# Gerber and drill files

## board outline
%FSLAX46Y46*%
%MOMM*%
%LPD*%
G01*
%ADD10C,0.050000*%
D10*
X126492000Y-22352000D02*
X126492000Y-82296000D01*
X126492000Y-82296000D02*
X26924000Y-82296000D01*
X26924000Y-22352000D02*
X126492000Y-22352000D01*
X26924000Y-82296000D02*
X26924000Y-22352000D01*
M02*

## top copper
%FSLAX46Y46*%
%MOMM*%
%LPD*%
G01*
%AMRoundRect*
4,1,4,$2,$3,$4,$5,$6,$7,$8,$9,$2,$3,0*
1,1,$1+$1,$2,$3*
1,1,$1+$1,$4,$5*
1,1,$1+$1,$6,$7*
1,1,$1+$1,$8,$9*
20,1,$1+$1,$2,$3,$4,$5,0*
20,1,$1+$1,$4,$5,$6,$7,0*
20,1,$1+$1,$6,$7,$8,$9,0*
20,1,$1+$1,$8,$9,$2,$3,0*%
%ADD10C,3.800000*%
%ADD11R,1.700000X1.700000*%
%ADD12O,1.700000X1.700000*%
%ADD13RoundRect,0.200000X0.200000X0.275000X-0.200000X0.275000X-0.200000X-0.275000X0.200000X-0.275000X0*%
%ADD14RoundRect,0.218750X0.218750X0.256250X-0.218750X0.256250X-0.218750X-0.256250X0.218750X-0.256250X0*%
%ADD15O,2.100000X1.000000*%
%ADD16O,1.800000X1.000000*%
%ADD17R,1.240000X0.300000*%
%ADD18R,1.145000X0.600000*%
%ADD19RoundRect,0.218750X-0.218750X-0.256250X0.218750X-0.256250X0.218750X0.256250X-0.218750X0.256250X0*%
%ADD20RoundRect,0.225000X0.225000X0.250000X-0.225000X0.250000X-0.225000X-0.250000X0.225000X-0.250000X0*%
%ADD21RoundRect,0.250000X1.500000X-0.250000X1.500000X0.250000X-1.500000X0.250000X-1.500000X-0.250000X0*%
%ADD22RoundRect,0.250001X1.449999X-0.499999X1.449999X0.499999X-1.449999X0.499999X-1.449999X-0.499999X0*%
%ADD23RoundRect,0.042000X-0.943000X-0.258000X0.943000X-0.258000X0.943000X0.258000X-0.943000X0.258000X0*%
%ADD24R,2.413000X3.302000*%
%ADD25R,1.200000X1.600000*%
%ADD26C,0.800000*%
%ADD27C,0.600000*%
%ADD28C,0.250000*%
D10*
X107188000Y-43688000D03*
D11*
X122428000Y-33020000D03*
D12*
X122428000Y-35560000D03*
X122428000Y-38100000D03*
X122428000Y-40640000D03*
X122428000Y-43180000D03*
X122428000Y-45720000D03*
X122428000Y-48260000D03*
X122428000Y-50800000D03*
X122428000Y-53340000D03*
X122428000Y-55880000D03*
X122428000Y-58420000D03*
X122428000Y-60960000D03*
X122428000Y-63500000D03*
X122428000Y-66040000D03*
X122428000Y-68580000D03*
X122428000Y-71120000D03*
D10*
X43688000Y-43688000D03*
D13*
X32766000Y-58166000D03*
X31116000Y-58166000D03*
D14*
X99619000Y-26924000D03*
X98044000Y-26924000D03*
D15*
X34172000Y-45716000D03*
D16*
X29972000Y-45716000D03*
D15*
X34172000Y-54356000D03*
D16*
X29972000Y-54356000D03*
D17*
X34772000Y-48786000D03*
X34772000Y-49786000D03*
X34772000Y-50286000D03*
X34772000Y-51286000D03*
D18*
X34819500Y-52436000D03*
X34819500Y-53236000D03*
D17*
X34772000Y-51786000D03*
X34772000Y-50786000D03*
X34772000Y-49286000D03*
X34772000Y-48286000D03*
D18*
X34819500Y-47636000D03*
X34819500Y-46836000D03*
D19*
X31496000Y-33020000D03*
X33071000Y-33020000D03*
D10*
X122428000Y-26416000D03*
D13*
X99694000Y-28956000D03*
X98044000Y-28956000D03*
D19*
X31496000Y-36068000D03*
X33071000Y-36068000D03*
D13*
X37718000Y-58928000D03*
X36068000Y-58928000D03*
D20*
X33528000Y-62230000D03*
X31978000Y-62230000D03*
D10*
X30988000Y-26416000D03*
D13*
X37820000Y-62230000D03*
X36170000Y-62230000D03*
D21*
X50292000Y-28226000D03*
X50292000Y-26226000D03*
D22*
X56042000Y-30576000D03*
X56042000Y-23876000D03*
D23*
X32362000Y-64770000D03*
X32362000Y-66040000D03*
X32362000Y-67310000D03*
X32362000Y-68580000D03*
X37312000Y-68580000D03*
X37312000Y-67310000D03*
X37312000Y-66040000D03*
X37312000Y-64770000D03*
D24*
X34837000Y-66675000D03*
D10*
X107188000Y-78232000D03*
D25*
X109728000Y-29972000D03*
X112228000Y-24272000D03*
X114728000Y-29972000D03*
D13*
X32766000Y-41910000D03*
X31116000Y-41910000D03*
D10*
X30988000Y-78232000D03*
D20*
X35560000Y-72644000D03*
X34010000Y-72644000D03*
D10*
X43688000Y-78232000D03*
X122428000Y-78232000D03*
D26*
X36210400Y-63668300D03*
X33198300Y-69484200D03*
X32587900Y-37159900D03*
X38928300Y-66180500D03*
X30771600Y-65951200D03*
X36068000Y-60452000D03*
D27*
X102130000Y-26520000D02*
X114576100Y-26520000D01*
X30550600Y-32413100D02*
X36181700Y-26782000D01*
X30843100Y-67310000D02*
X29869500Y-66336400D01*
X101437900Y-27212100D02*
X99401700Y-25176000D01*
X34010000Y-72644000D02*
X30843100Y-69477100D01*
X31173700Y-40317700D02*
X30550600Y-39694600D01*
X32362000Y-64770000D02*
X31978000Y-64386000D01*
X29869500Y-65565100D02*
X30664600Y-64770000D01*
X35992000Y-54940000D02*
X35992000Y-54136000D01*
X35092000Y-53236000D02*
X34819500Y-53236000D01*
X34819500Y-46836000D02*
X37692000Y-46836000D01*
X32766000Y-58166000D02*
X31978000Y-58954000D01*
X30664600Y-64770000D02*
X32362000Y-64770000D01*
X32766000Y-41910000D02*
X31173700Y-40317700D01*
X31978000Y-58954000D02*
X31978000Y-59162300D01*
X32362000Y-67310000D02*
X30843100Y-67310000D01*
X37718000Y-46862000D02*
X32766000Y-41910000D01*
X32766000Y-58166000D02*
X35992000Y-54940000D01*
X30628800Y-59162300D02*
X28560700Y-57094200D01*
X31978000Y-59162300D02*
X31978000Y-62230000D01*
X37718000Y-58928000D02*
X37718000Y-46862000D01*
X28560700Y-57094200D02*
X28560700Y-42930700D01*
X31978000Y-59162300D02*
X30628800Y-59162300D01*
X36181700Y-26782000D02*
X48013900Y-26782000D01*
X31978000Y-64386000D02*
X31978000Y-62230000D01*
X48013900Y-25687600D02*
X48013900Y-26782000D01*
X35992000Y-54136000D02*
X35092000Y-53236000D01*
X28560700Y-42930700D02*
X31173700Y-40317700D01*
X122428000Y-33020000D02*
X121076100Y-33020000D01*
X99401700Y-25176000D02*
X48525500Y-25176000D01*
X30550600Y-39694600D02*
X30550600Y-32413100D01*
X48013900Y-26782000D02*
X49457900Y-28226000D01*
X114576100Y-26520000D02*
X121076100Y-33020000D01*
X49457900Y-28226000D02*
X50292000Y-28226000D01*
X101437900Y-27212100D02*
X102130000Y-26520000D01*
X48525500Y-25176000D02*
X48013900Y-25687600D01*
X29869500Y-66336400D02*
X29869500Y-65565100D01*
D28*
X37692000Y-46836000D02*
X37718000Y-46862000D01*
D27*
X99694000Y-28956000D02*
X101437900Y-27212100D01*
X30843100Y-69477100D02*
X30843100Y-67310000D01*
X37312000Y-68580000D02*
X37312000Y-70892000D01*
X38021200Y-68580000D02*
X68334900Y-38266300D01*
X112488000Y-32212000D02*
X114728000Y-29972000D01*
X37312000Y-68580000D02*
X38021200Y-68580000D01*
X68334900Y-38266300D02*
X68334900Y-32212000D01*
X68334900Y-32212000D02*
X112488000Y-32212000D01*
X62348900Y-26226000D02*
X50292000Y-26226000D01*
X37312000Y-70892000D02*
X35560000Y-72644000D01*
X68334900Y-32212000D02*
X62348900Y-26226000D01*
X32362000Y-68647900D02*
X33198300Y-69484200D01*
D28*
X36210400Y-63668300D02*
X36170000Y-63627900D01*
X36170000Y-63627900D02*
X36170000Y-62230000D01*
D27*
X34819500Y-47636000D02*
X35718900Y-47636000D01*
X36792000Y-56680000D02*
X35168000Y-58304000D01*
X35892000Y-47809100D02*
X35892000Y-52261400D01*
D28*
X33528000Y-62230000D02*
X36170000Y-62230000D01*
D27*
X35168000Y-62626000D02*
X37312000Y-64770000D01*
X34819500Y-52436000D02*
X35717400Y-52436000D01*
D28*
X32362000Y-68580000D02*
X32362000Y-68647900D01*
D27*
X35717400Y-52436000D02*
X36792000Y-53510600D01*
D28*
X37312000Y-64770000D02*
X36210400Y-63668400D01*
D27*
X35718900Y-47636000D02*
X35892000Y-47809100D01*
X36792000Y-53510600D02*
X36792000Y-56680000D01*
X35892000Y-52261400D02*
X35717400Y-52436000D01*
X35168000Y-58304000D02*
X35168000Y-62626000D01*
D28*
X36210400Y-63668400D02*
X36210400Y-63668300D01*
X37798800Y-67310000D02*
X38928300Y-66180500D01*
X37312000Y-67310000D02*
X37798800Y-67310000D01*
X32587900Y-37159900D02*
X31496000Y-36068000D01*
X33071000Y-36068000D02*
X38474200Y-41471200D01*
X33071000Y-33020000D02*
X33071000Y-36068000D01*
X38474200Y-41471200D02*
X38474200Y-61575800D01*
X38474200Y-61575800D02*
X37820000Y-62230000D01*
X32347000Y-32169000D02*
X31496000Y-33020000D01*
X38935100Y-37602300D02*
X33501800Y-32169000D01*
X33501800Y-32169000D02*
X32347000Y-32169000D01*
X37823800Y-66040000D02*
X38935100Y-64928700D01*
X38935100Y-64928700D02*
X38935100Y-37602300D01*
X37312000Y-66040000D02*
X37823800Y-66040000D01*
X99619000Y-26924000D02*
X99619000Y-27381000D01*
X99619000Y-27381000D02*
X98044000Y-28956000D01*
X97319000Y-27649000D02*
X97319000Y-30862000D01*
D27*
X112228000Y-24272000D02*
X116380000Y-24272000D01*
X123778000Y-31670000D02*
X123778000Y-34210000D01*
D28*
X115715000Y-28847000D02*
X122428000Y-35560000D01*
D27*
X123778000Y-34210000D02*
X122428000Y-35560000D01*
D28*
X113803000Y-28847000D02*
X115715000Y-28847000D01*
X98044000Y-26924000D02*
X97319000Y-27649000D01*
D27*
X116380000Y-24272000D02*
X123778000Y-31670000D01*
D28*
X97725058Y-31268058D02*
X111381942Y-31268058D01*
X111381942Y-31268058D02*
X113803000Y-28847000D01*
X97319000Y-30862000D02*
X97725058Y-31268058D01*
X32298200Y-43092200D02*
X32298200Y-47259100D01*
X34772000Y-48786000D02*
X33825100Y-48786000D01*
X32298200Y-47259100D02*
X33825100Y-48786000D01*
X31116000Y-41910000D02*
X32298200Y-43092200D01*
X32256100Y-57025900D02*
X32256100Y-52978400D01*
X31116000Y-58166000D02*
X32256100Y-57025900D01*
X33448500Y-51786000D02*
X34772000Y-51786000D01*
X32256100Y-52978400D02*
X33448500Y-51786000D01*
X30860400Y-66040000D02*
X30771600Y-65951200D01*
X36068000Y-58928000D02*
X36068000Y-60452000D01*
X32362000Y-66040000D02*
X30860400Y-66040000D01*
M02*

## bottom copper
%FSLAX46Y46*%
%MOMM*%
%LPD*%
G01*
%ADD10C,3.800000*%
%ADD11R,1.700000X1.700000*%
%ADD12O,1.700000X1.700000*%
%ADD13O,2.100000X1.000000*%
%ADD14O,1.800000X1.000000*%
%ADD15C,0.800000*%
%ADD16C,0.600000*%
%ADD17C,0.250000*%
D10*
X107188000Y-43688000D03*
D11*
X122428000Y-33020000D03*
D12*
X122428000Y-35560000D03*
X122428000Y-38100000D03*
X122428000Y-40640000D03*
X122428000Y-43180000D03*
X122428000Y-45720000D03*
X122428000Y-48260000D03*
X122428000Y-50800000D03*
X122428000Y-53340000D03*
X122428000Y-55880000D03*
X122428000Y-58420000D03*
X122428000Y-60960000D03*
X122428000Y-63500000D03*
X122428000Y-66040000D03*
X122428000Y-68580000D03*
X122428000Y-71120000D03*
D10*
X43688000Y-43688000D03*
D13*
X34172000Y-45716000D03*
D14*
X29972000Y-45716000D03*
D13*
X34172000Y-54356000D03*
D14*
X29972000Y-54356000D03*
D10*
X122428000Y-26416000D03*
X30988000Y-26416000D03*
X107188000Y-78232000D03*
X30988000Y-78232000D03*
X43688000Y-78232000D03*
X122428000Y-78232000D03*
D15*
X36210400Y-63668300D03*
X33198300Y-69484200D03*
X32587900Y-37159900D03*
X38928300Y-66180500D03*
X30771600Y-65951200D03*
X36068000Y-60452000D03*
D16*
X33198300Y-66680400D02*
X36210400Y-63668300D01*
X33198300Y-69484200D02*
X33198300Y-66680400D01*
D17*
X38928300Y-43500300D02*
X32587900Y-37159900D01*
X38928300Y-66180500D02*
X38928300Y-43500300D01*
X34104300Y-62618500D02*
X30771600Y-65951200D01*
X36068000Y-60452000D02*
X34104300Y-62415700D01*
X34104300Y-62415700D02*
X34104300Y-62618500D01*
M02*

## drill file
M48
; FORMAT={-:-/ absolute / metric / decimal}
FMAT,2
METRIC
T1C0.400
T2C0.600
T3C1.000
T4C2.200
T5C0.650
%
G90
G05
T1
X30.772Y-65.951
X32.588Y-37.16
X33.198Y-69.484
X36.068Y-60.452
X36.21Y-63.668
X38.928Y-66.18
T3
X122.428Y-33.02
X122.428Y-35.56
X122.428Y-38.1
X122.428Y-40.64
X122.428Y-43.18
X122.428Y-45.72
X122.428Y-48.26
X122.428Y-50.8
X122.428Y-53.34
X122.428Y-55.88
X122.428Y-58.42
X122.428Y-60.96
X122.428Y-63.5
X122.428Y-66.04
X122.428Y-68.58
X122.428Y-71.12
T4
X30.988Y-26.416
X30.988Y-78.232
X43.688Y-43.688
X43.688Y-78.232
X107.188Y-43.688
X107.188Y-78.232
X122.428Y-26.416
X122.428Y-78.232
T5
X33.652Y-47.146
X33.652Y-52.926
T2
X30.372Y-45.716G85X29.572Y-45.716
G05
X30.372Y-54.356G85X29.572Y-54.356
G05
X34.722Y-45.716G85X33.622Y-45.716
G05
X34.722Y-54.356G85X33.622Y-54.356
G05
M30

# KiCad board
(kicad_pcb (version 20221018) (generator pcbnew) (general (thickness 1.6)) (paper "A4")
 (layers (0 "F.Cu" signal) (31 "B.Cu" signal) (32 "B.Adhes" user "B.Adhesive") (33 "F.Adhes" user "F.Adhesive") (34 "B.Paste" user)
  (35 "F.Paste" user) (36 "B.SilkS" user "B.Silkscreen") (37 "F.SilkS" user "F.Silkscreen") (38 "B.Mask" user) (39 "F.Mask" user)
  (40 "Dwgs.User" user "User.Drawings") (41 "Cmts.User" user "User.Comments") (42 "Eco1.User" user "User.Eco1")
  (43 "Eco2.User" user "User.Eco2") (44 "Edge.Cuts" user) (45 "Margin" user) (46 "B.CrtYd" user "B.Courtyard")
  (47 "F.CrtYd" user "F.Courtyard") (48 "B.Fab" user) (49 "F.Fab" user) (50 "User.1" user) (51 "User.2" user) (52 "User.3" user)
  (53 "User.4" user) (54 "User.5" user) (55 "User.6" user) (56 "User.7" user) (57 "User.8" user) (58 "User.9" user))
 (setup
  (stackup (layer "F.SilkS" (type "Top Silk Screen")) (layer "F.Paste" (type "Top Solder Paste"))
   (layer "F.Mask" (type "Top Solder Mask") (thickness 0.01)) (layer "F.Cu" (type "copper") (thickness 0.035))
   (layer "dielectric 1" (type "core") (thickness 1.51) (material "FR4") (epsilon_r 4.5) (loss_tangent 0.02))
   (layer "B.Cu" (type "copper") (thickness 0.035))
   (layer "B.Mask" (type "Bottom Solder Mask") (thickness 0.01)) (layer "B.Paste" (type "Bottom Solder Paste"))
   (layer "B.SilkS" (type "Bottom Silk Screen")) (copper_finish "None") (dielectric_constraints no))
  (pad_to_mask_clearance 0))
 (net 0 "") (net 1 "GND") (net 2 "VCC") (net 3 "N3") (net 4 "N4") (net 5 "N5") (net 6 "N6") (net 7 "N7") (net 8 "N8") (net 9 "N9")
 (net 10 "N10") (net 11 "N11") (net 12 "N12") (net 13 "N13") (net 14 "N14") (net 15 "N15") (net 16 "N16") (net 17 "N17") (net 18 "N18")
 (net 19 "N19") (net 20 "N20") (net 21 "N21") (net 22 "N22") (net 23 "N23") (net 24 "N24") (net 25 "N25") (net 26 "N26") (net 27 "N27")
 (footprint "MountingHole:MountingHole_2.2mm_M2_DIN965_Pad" (layer "F.Cu") (at 107.188 43.688)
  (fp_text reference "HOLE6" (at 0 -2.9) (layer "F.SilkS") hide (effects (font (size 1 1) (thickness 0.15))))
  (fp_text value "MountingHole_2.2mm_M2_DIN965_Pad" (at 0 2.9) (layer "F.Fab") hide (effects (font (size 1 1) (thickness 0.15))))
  (pad "1" thru_hole circle (at 0 0) (size 3.8 3.8) (drill 2.2) (layers "*.Cu" "*.Mask")))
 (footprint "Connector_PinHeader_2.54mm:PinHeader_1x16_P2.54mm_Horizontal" (layer "F.Cu") (at 122.428 33.02)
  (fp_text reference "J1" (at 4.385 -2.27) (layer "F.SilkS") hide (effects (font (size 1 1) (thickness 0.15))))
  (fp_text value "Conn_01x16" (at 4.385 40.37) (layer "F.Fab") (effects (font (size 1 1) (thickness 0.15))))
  (pad "1" thru_hole rect (at 0 0) (size 1.7 1.7) (drill 1) (layers "*.Cu" "*.Mask") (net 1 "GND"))
  (pad "2" thru_hole oval (at 0 2.54) (size 1.7 1.7) (drill 1) (layers "*.Cu" "*.Mask") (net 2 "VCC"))
  (pad "3" thru_hole oval (at 0 5.08) (size 1.7 1.7) (drill 1) (layers "*.Cu" "*.Mask") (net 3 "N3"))
  (pad "4" thru_hole oval (at 0 7.62) (size 1.7 1.7) (drill 1) (layers "*.Cu" "*.Mask") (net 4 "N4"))
  (pad "5" thru_hole oval (at 0 10.16) (size 1.7 1.7) (drill 1) (layers "*.Cu" "*.Mask") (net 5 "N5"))
  (pad "6" thru_hole oval (at 0 12.7) (size 1.7 1.7) (drill 1) (layers "*.Cu" "*.Mask") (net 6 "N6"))
  (pad "7" thru_hole oval (at 0 15.24) (size 1.7 1.7) (drill 1) (layers "*.Cu" "*.Mask") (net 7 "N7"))
  (pad "8" thru_hole oval (at 0 17.78) (size 1.7 1.7) (drill 1) (layers "*.Cu" "*.Mask") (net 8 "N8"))
  (pad "9" thru_hole oval (at 0 20.32) (size 1.7 1.7) (drill 1) (layers "*.Cu" "*.Mask") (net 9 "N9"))
  (pad "10" thru_hole oval (at 0 22.86) (size 1.7 1.7) (drill 1) (layers "*.Cu" "*.Mask") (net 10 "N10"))
  (pad "11" thru_hole oval (at 0 25.4) (size 1.7 1.7) (drill 1) (layers "*.Cu" "*.Mask") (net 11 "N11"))
  (pad "12" thru_hole oval (at 0 27.94) (size 1.7 1.7) (drill 1) (layers "*.Cu" "*.Mask") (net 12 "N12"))
  (pad "13" thru_hole oval (at 0 30.48) (size 1.7 1.7) (drill 1) (layers "*.Cu" "*.Mask") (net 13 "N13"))
  (pad "14" thru_hole oval (at 0 33.02) (size 1.7 1.7) (drill 1) (layers "*.Cu" "*.Mask") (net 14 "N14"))
  (pad "15" thru_hole oval (at 0 35.56) (size 1.7 1.7) (drill 1) (layers "*.Cu" "*.Mask") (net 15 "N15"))
  (pad "16" thru_hole oval (at 0 38.1) (size 1.7 1.7) (drill 1) (layers "*.Cu" "*.Mask") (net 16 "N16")))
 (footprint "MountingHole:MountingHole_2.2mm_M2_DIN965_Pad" (layer "F.Cu") (at 43.688 43.688)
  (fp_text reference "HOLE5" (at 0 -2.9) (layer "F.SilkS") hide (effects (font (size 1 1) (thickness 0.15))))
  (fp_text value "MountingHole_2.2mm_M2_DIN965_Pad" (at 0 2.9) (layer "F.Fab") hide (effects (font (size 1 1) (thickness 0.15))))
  (pad "1" thru_hole circle (at 0 0) (size 3.8 3.8) (drill 2.2) (layers "*.Cu" "*.Mask")))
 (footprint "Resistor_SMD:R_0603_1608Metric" (layer "F.Cu") (at 31.941 58.166 180)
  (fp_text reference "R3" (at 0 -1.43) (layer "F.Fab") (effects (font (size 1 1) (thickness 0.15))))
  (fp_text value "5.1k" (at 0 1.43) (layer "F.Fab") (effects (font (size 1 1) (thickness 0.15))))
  (pad "1" smd roundrect (at -0.825 0 180) (size 0.8 0.95) (layers "F.Cu" "F.Paste" "F.Mask") (roundrect_rratio 0.25) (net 1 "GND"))
  (pad "2" smd roundrect (at 0.825 0 180) (size 0.8 0.95) (layers "F.Cu" "F.Paste" "F.Mask") (roundrect_rratio 0.25) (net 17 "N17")))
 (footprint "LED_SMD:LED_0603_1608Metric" (layer "F.Cu") (at 98.8315 26.924 180)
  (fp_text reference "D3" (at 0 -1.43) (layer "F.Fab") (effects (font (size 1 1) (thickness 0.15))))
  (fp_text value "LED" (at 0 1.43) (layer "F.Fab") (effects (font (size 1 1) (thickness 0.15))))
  (pad "1" smd roundrect (at -0.7875 0 180) (size 0.875 0.95) (layers "F.Cu" "F.Paste" "F.Mask") (roundrect_rratio 0.25) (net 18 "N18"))
  (pad "2" smd roundrect (at 0.7875 0 180) (size 0.875 0.95) (layers "F.Cu" "F.Paste" "F.Mask") (roundrect_rratio 0.25) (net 2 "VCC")))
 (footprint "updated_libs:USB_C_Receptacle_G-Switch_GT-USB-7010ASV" (layer "F.Cu") (at 31.047 50.036 -90)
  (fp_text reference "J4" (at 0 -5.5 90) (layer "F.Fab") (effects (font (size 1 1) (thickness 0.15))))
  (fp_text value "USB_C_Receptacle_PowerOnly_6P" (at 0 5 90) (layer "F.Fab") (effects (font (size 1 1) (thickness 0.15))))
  (pad "" thru_hole oval (at -4.32 -3.125 270) (size 1 2.1) (drill oval 0.6 1.7) (layers "*.Cu" "*.Mask"))
  (pad "" thru_hole oval (at -4.32 1.075 270) (size 1 1.8) (drill oval 0.6 1.4) (layers "*.Cu" "*.Mask"))
  (pad "" np_thru_hole circle (at -2.89 -2.605 270) (size 0.65 0.65) (drill 0.65) (layers "*.Cu" "*.Mask"))
  (pad "" np_thru_hole circle (at 2.89 -2.605 270) (size 0.65 0.65) (drill 0.65) (layers "*.Cu" "*.Mask"))
  (pad "" thru_hole oval (at 4.32 -3.125 270) (size 1 2.1) (drill oval 0.6 1.7) (layers "*.Cu" "*.Mask"))
  (pad "" thru_hole oval (at 4.32 1.075 270) (size 1 1.8) (drill oval 0.6 1.4) (layers "*.Cu" "*.Mask"))
  (pad "A5" smd rect (at -1.25 -3.725 270) (size 0.3 1.24) (layers "F.Cu" "F.Paste" "F.Mask") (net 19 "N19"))
  (pad "A6" smd rect (at -0.25 -3.725 270) (size 0.3 1.24) (layers "F.Cu" "F.Paste" "F.Mask"))
  (pad "A7" smd rect (at 0.25 -3.725 270) (size 0.3 1.24) (layers "F.Cu" "F.Paste" "F.Mask"))
  (pad "A8" smd rect (at 1.25 -3.725 270) (size 0.3 1.24) (layers "F.Cu" "F.Paste" "F.Mask"))
  (pad "A9" smd rect (at 2.4 -3.7725 270) (size 0.6 1.145) (layers "F.Cu" "F.Paste" "F.Mask") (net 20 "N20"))
  (pad "A12" smd rect (at 3.2 -3.7725 270) (size 0.6 1.145) (layers "F.Cu" "F.Paste" "F.Mask") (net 1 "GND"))
  (pad "B5" smd rect (at 1.75 -3.725 270) (size 0.3 1.24) (layers "F.Cu" "F.Paste" "F.Mask") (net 17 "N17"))
  (pad "B6" smd rect (at 0.75 -3.725 270) (size 0.3 1.24) (layers "F.Cu" "F.Paste" "F.Mask"))
  (pad "B7" smd rect (at -0.75 -3.725 270) (size 0.3 1.24) (layers "F.Cu" "F.Paste" "F.Mask"))
  (pad "B8" smd rect (at -1.75 -3.725 270) (size 0.3 1.24) (layers "F.Cu" "F.Paste" "F.Mask"))
  (pad "B9" smd rect (at -2.4 -3.7725 270) (size 0.6 1.145) (layers "F.Cu" "F.Paste" "F.Mask") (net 20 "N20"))
  (pad "B12" smd rect (at -3.2 -3.7725 270) (size 0.6 1.145) (layers "F.Cu" "F.Paste" "F.Mask") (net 1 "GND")))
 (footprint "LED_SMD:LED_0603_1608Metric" (layer "F.Cu") (at 32.2835 33.02)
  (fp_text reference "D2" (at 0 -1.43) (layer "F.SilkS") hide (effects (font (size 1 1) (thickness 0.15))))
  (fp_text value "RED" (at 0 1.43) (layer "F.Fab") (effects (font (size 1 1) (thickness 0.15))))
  (pad "1" smd roundrect (at -0.7875 0) (size 0.875 0.95) (layers "F.Cu" "F.Paste" "F.Mask") (roundrect_rratio 0.25) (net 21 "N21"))
  (pad "2" smd roundrect (at 0.7875 0) (size 0.875 0.95) (layers "F.Cu" "F.Paste" "F.Mask") (roundrect_rratio 0.25) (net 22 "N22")))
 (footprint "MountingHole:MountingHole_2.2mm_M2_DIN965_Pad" (layer "F.Cu") (at 122.428 26.416)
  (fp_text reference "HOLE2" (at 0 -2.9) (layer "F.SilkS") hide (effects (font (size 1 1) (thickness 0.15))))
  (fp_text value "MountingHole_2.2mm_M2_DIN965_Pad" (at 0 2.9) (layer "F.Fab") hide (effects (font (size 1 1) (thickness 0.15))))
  (pad "1" thru_hole circle (at 0 0) (size 3.8 3.8) (drill 2.2) (layers "*.Cu" "*.Mask")))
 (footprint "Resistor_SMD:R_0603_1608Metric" (layer "F.Cu") (at 98.869 28.956 180)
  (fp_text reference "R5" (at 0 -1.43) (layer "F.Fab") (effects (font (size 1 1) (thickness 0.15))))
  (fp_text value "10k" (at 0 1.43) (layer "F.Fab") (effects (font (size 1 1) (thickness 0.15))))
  (pad "1" smd roundrect (at -0.825 0 180) (size 0.8 0.95) (layers "F.Cu" "F.Paste" "F.Mask") (roundrect_rratio 0.25) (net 1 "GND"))
  (pad "2" smd roundrect (at 0.825 0 180) (size 0.8 0.95) (layers "F.Cu" "F.Paste" "F.Mask") (roundrect_rratio 0.25) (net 18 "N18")))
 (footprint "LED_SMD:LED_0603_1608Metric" (layer "F.Cu") (at 32.2835 36.068)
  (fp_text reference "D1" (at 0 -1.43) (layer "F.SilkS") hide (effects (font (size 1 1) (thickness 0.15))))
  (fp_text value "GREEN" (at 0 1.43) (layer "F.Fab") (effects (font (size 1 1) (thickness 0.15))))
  (pad "1" smd roundrect (at -0.7875 0) (size 0.875 0.95) (layers "F.Cu" "F.Paste" "F.Mask") (roundrect_rratio 0.25) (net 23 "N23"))
  (pad "2" smd roundrect (at 0.7875 0) (size 0.875 0.95) (layers "F.Cu" "F.Paste" "F.Mask") (roundrect_rratio 0.25) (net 22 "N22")))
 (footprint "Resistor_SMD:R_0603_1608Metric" (layer "F.Cu") (at 36.893 58.928 180)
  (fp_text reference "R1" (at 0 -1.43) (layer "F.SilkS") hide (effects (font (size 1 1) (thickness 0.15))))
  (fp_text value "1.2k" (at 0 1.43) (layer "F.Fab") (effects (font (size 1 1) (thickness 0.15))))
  (pad "1" smd roundrect (at -0.825 0 180) (size 0.8 0.95) (layers "F.Cu" "F.Paste" "F.Mask") (roundrect_rratio 0.25) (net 1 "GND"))
  (pad "2" smd roundrect (at 0.825 0 180) (size 0.8 0.95) (layers "F.Cu" "F.Paste" "F.Mask") (roundrect_rratio 0.25) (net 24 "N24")))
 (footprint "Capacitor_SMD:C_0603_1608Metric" (layer "F.Cu") (at 32.753 62.23 180)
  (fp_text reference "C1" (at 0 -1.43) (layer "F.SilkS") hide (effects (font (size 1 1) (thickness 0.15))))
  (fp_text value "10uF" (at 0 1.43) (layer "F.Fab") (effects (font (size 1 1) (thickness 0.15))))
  (pad "1" smd roundrect (at -0.775 0 180) (size 0.9 0.95) (layers "F.Cu" "F.Paste" "F.Mask") (roundrect_rratio 0.25) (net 20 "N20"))
  (pad "2" smd roundrect (at 0.775 0 180) (size 0.9 0.95) (layers "F.Cu" "F.Paste" "F.Mask") (roundrect_rratio 0.25) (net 1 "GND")))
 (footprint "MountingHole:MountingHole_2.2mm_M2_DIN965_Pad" (layer "F.Cu") (at 30.988 26.416)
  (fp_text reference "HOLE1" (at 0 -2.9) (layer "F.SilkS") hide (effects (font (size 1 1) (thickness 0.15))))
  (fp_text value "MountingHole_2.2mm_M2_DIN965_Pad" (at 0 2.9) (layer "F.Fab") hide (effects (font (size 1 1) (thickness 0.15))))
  (pad "1" thru_hole circle (at 0 0) (size 3.8 3.8) (drill 2.2) (layers "*.Cu" "*.Mask")))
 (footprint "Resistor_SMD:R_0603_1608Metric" (layer "F.Cu") (at 36.995 62.23 180)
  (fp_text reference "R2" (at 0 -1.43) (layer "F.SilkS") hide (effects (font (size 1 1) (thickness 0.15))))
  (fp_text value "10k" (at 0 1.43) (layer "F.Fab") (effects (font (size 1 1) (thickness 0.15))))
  (pad "1" smd roundrect (at -0.825 0 180) (size 0.8 0.95) (layers "F.Cu" "F.Paste" "F.Mask") (roundrect_rratio 0.25) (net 22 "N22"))
  (pad "2" smd roundrect (at 0.825 0 180) (size 0.8 0.95) (layers "F.Cu" "F.Paste" "F.Mask") (roundrect_rratio 0.25) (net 20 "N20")))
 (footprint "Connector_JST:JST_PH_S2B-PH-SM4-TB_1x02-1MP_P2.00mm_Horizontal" (layer "F.Cu") (at 53.142 27.226 90)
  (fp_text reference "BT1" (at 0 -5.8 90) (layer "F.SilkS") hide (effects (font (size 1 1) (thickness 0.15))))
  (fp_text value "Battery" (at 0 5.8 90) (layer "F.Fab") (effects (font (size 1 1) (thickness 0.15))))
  (pad "1" smd roundrect (at -1 -2.85 90) (size 1 3.5) (layers "F.Cu" "F.Paste" "F.Mask") (roundrect_rratio 0.25) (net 1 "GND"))
  (pad "2" smd roundrect (at 1 -2.85 90) (size 1 3.5) (layers "F.Cu" "F.Paste" "F.Mask") (roundrect_rratio 0.25) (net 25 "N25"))
  (pad "MP" smd roundrect (at -3.35 2.9 90) (size 1.5 3.4) (layers "F.Cu" "F.Paste" "F.Mask") (roundrect_rratio 0.1666673333))
  (pad "MP" smd roundrect (at 3.35 2.9 90) (size 1.5 3.4) (layers "F.Cu" "F.Paste" "F.Mask") (roundrect_rratio 0.1666673333)))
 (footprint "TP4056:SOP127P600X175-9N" (layer "F.Cu") (at 34.837 66.675)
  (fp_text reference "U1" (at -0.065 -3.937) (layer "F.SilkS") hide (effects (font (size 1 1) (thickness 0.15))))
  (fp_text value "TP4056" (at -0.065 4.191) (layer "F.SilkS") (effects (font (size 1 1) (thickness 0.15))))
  (pad "1" smd roundrect (at -2.475 -1.905) (size 1.97 0.6) (layers "F.Cu" "F.Paste" "F.Mask") (roundrect_rratio 0.07) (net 1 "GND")
   (solder_mask_margin 0.102))
  (pad "2" smd roundrect (at -2.475 -0.635) (size 1.97 0.6) (layers "F.Cu" "F.Paste" "F.Mask") (roundrect_rratio 0.07) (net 24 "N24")
   (solder_mask_margin 0.102))
  (pad "3" smd roundrect (at -2.475 0.635) (size 1.97 0.6) (layers "F.Cu" "F.Paste" "F.Mask") (roundrect_rratio 0.07) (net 1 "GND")
   (solder_mask_margin 0.102))
  (pad "4" smd roundrect (at -2.475 1.905) (size 1.97 0.6) (layers "F.Cu" "F.Paste" "F.Mask") (roundrect_rratio 0.07) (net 20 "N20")
   (solder_mask_margin 0.102))
  (pad "5" smd roundrect (at 2.475 1.905) (size 1.97 0.6) (layers "F.Cu" "F.Paste" "F.Mask") (roundrect_rratio 0.07) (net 25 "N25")
   (solder_mask_margin 0.102))
  (pad "6" smd roundrect (at 2.475 0.635) (size 1.97 0.6) (layers "F.Cu" "F.Paste" "F.Mask") (roundrect_rratio 0.07) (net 23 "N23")
   (solder_mask_margin 0.102))
  (pad "7" smd roundrect (at 2.475 -0.635) (size 1.97 0.6) (layers "F.Cu" "F.Paste" "F.Mask") (roundrect_rratio 0.07) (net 21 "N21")
   (solder_mask_margin 0.102))
  (pad "8" smd roundrect (at 2.475 -1.905) (size 1.97 0.6) (layers "F.Cu" "F.Paste" "F.Mask") (roundrect_rratio 0.07) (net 20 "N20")
   (solder_mask_margin 0.102))
  (pad "9" smd rect (at 0 0) (size 2.413 3.302) (layers "F.Cu" "F.Mask") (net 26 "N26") (solder_mask_margin 0.102)))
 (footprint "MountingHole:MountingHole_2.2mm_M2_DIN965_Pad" (layer "F.Cu") (at 107.188 78.232)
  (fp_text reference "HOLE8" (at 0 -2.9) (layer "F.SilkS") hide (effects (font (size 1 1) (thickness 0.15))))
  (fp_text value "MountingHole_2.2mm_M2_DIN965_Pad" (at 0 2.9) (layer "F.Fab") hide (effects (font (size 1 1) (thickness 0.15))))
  (pad "1" thru_hole circle (at 0 0) (size 3.8 3.8) (drill 2.2) (layers "*.Cu" "*.Mask")))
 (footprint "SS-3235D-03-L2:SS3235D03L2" (layer "F.Cu") (at 112.228 27.122)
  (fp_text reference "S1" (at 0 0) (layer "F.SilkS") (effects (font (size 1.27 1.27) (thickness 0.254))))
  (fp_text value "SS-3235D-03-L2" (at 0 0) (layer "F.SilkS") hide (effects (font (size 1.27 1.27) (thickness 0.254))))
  (pad "1" smd rect (at -2.5 2.85) (size 1.2 1.6) (layers "F.Cu" "F.Paste" "F.Mask") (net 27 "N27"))
  (pad "2" smd rect (at 0 -2.85) (size 1.2 1.6) (layers "F.Cu" "F.Paste" "F.Mask") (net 2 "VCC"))
  (pad "3" smd rect (at 2.5 2.85) (size 1.2 1.6) (layers "F.Cu" "F.Paste" "F.Mask") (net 25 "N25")))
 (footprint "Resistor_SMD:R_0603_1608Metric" (layer "F.Cu") (at 31.941 41.91 180)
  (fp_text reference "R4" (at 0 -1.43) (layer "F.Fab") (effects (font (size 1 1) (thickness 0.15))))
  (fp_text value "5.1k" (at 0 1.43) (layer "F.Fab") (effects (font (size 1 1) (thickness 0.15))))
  (pad "1" smd roundrect (at -0.825 0 180) (size 0.8 0.95) (layers "F.Cu" "F.Paste" "F.Mask") (roundrect_rratio 0.25) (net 1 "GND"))
  (pad "2" smd roundrect (at 0.825 0 180) (size 0.8 0.95) (layers "F.Cu" "F.Paste" "F.Mask") (roundrect_rratio 0.25) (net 19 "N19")))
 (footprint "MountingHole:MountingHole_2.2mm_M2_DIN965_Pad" (layer "F.Cu") (at 30.988 78.232)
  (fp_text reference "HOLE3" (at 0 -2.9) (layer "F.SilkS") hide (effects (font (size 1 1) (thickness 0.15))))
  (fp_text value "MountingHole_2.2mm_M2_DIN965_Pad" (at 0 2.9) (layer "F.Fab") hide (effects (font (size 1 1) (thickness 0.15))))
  (pad "1" thru_hole circle (at 0 0) (size 3.8 3.8) (drill 2.2) (layers "*.Cu" "*.Mask")))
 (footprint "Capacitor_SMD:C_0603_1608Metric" (layer "F.Cu") (at 34.785 72.644 180)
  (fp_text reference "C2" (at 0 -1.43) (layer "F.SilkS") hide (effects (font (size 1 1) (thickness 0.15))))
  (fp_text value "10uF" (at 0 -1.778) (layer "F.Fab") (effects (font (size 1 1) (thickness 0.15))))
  (pad "1" smd roundrect (at -0.775 0 180) (size 0.9 0.95) (layers "F.Cu" "F.Paste" "F.Mask") (roundrect_rratio 0.25) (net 25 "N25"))
  (pad "2" smd roundrect (at 0.775 0 180) (size 0.9 0.95) (layers "F.Cu" "F.Paste" "F.Mask") (roundrect_rratio 0.25) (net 1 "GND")))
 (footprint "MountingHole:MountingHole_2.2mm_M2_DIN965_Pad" (layer "F.Cu") (at 43.688 78.232)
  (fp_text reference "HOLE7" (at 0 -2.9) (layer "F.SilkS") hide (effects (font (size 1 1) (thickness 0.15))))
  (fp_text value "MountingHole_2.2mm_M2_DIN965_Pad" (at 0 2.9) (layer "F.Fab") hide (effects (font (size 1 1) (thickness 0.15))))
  (pad "1" thru_hole circle (at 0 0) (size 3.8 3.8) (drill 2.2) (layers "*.Cu" "*.Mask")))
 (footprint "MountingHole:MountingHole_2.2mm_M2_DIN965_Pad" (layer "F.Cu") (at 122.428 78.232)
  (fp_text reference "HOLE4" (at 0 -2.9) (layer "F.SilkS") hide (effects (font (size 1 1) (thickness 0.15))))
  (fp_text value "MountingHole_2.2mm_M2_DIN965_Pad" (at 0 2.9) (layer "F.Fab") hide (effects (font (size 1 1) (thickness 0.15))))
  (pad "1" thru_hole circle (at 0 0) (size 3.8 3.8) (drill 2.2) (layers "*.Cu" "*.Mask")))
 (gr_line (start 126.492 22.352) (end 126.492 82.296) (stroke (width 0.05) (type solid)) (layer "Edge.Cuts"))
 (gr_line (start 126.492 82.296) (end 26.924 82.296) (stroke (width 0.05) (type solid)) (layer "Edge.Cuts"))
 (gr_line (start 26.924 22.352) (end 126.492 22.352) (stroke (width 0.05) (type solid)) (layer "Edge.Cuts"))
 (gr_line (start 26.924 82.296) (end 26.924 22.352) (stroke (width 0.05) (type solid)) (layer "Edge.Cuts"))
 (segment (start 102.13 26.52) (end 114.5761 26.52) (width 0.6) (layer "F.Cu") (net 1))
 (segment (start 30.5506 32.4131) (end 36.1817 26.782) (width 0.6) (layer "F.Cu") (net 1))
 (segment (start 30.8431 67.31) (end 29.8695 66.3364) (width 0.6) (layer "F.Cu") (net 1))
 (segment (start 101.4379 27.2121) (end 99.4017 25.176) (width 0.6) (layer "F.Cu") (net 1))
 (segment (start 34.01 72.644) (end 30.8431 69.4771) (width 0.6) (layer "F.Cu") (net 1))
 (segment (start 31.1737 40.3177) (end 30.5506 39.6946) (width 0.6) (layer "F.Cu") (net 1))
 (segment (start 32.362 64.77) (end 31.978 64.386) (width 0.6) (layer "F.Cu") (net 1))
 (segment (start 29.8695 65.5651) (end 30.6646 64.77) (width 0.6) (layer "F.Cu") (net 1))
 (segment (start 35.992 54.94) (end 35.992 54.136) (width 0.6) (layer "F.Cu") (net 1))
 (segment (start 35.092 53.236) (end 34.8195 53.236) (width 0.6) (layer "F.Cu") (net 1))
 (segment (start 34.8195 46.836) (end 37.692 46.836) (width 0.6) (layer "F.Cu") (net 1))
 (segment (start 32.766 58.166) (end 31.978 58.954) (width 0.6) (layer "F.Cu") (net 1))
 (segment (start 30.6646 64.77) (end 32.362 64.77) (width 0.6) (layer "F.Cu") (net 1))
 (segment (start 32.766 41.91) (end 31.1737 40.3177) (width 0.6) (layer "F.Cu") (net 1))
 (segment (start 31.978 58.954) (end 31.978 59.1623) (width 0.6) (layer "F.Cu") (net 1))
 (segment (start 32.362 67.31) (end 30.8431 67.31) (width 0.6) (layer "F.Cu") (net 1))
 (segment (start 37.718 46.862) (end 32.766 41.91) (width 0.6) (layer "F.Cu") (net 1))
 (segment (start 32.766 58.166) (end 35.992 54.94) (width 0.6) (layer "F.Cu") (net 1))
 (segment (start 30.6288 59.1623) (end 28.5607 57.0942) (width 0.6) (layer "F.Cu") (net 1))
 (segment (start 31.978 59.1623) (end 31.978 62.23) (width 0.6) (layer "F.Cu") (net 1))
 (segment (start 37.718 58.928) (end 37.718 46.862) (width 0.6) (layer "F.Cu") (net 1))
 (segment (start 28.5607 57.0942) (end 28.5607 42.9307) (width 0.6) (layer "F.Cu") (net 1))
 (segment (start 31.978 59.1623) (end 30.6288 59.1623) (width 0.6) (layer "F.Cu") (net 1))
 (segment (start 36.1817 26.782) (end 48.0139 26.782) (width 0.6) (layer "F.Cu") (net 1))
 (segment (start 31.978 64.386) (end 31.978 62.23) (width 0.6) (layer "F.Cu") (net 1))
 (segment (start 48.0139 25.6876) (end 48.0139 26.782) (width 0.6) (layer "F.Cu") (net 1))
 (segment (start 35.992 54.136) (end 35.092 53.236) (width 0.6) (layer "F.Cu") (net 1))
 (segment (start 28.5607 42.9307) (end 31.1737 40.3177) (width 0.6) (layer "F.Cu") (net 1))
 (segment (start 122.428 33.02) (end 121.0761 33.02) (width 0.6) (layer "F.Cu") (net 1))
 (segment (start 99.4017 25.176) (end 48.5255 25.176) (width 0.6) (layer "F.Cu") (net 1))
 (segment (start 30.5506 39.6946) (end 30.5506 32.4131) (width 0.6) (layer "F.Cu") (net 1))
 (segment (start 48.0139 26.782) (end 49.4579 28.226) (width 0.6) (layer "F.Cu") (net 1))
 (segment (start 114.5761 26.52) (end 121.0761 33.02) (width 0.6) (layer "F.Cu") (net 1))
 (segment (start 49.4579 28.226) (end 50.292 28.226) (width 0.6) (layer "F.Cu") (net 1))
 (segment (start 101.4379 27.2121) (end 102.13 26.52) (width 0.6) (layer "F.Cu") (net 1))
 (segment (start 48.5255 25.176) (end 48.0139 25.6876) (width 0.6) (layer "F.Cu") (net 1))
 (segment (start 29.8695 66.3364) (end 29.8695 65.5651) (width 0.6) (layer "F.Cu") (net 1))
 (segment (start 37.692 46.836) (end 37.718 46.862) (width 0.25) (layer "F.Cu") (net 1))
 (segment (start 99.694 28.956) (end 101.4379 27.2121) (width 0.6) (layer "F.Cu") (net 1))
 (segment (start 30.8431 69.4771) (end 30.8431 67.31) (width 0.6) (layer "F.Cu") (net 1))
 (segment (start 37.312 68.58) (end 37.312 70.892) (width 0.6) (layer "F.Cu") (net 25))
 (segment (start 38.0212 68.58) (end 68.3349 38.2663) (width 0.6) (layer "F.Cu") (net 25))
 (segment (start 112.488 32.212) (end 114.728 29.972) (width 0.6) (layer "F.Cu") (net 25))
 (segment (start 37.312 68.58) (end 38.0212 68.58) (width 0.6) (layer "F.Cu") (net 25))
 (segment (start 68.3349 38.2663) (end 68.3349 32.212) (width 0.6) (layer "F.Cu") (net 25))
 (segment (start 68.3349 32.212) (end 112.488 32.212) (width 0.6) (layer "F.Cu") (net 25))
 (segment (start 62.3489 26.226) (end 50.292 26.226) (width 0.6) (layer "F.Cu") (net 25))
 (segment (start 37.312 70.892) (end 35.56 72.644) (width 0.6) (layer "F.Cu") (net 25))
 (segment (start 68.3349 32.212) (end 62.3489 26.226) (width 0.6) (layer "F.Cu") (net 25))
 (segment (start 32.362 68.6479) (end 33.1983 69.4842) (width 0.6) (layer "F.Cu") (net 20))
 (segment (start 36.2104 63.6683) (end 36.17 63.6279) (width 0.25) (layer "F.Cu") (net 20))
 (segment (start 36.17 63.6279) (end 36.17 62.23) (width 0.25) (layer "F.Cu") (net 20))
 (segment (start 34.8195 47.636) (end 35.7189 47.636) (width 0.6) (layer "F.Cu") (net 20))
 (segment (start 36.792 56.68) (end 35.168 58.304) (width 0.6) (layer "F.Cu") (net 20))
 (segment (start 35.892 47.8091) (end 35.892 52.2614) (width 0.6) (layer "F.Cu") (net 20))
 (segment (start 33.528 62.23) (end 36.17 62.23) (width 0.25) (layer "F.Cu") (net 20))
 (segment (start 35.168 62.626) (end 37.312 64.77) (width 0.6) (layer "F.Cu") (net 20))
 (segment (start 34.8195 52.436) (end 35.7174 52.436) (width 0.6) (layer "F.Cu") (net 20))
 (segment (start 32.362 68.58) (end 32.362 68.6479) (width 0.25) (layer "F.Cu") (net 20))
 (segment (start 35.7174 52.436) (end 36.792 53.5106) (width 0.6) (layer "F.Cu") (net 20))
 (segment (start 37.312 64.77) (end 36.2104 63.6684) (width 0.25) (layer "F.Cu") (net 20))
 (segment (start 35.7189 47.636) (end 35.892 47.8091) (width 0.6) (layer "F.Cu") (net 20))
 (segment (start 36.792 53.5106) (end 36.792 56.68) (width 0.6) (layer "F.Cu") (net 20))
 (segment (start 35.892 52.2614) (end 35.7174 52.436) (width 0.6) (layer "F.Cu") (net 20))
 (segment (start 35.168 58.304) (end 35.168 62.626) (width 0.6) (layer "F.Cu") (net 20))
 (segment (start 36.2104 63.6684) (end 36.2104 63.6683) (width 0.25) (layer "F.Cu") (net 20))
 (via (at 36.2104 63.6683) (size 0.8) (drill 0.4) (layers "F.Cu" "B.Cu") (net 20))
 (via (at 33.1983 69.4842) (size 0.8) (drill 0.4) (layers "F.Cu" "B.Cu") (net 20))
 (segment (start 33.1983 66.6804) (end 36.2104 63.6683) (width 0.6) (layer "B.Cu") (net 20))
 (segment (start 33.1983 69.4842) (end 33.1983 66.6804) (width 0.6) (layer "B.Cu") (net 20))
 (segment (start 37.7988 67.31) (end 38.9283 66.1805) (width 0.25) (layer "F.Cu") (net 23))
 (segment (start 37.312 67.31) (end 37.7988 67.31) (width 0.25) (layer "F.Cu") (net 23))
 (segment (start 32.5879 37.1599) (end 31.496 36.068) (width 0.25) (layer "F.Cu") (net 23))
 (via (at 32.5879 37.1599) (size 0.8) (drill 0.4) (layers "F.Cu" "B.Cu") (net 23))
 (via (at 38.9283 66.1805) (size 0.8) (drill 0.4) (layers "F.Cu" "B.Cu") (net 23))
 (segment (start 38.9283 43.5003) (end 32.5879 37.1599) (width 0.25) (layer "B.Cu") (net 23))
 (segment (start 38.9283 66.1805) (end 38.9283 43.5003) (width 0.25) (layer "B.Cu") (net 23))
 (segment (start 33.071 36.068) (end 38.4742 41.4712) (width 0.25) (layer "F.Cu") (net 22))
 (segment (start 33.071 33.02) (end 33.071 36.068) (width 0.25) (layer "F.Cu") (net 22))
 (segment (start 38.4742 41.4712) (end 38.4742 61.5758) (width 0.25) (layer "F.Cu") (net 22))
 (segment (start 38.4742 61.5758) (end 37.82 62.23) (width 0.25) (layer "F.Cu") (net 22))
 (segment (start 32.347 32.169) (end 31.496 33.02) (width 0.25) (layer "F.Cu") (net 21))
 (segment (start 38.9351 37.6023) (end 33.5018 32.169) (width 0.25) (layer "F.Cu") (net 21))
 (segment (start 33.5018 32.169) (end 32.347 32.169) (width 0.25) (layer "F.Cu") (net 21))
 (segment (start 37.8238 66.04) (end 38.9351 64.9287) (width 0.25) (layer "F.Cu") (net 21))
 (segment (start 38.9351 64.9287) (end 38.9351 37.6023) (width 0.25) (layer "F.Cu") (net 21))
 (segment (start 37.312 66.04) (end 37.8238 66.04) (width 0.25) (layer "F.Cu") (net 21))
 (segment (start 99.619 26.924) (end 99.619 27.381) (width 0.25) (layer "F.Cu") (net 18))
 (segment (start 99.619 27.381) (end 98.044 28.956) (width 0.25) (layer "F.Cu") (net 18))
 (segment (start 97.319 27.649) (end 97.319 30.862) (width 0.25) (layer "F.Cu") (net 2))
 (segment (start 112.228 24.272) (end 116.38 24.272) (width 0.6) (layer "F.Cu") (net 2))
 (segment (start 123.778 31.67) (end 123.778 34.21) (width 0.6) (layer "F.Cu") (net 2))
 (segment (start 115.715 28.847) (end 122.428 35.56) (width 0.25) (layer "F.Cu") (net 2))
 (segment (start 123.778 34.21) (end 122.428 35.56) (width 0.6) (layer "F.Cu") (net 2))
 (segment (start 113.803 28.847) (end 115.715 28.847) (width 0.25) (layer "F.Cu") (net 2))
 (segment (start 98.044 26.924) (end 97.319 27.649) (width 0.25) (layer "F.Cu") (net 2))
 (segment (start 116.38 24.272) (end 123.778 31.67) (width 0.6) (layer "F.Cu") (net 2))
 (segment (start 97.725058 31.268058) (end 111.381942 31.268058) (width 0.25) (layer "F.Cu") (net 2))
 (segment (start 111.381942 31.268058) (end 113.803 28.847) (width 0.25) (layer "F.Cu") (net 2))
 (segment (start 97.319 30.862) (end 97.725058 31.268058) (width 0.25) (layer "F.Cu") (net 2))
 (segment (start 32.2982 43.0922) (end 32.2982 47.2591) (width 0.25) (layer "F.Cu") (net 19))
 (segment (start 34.772 48.786) (end 33.8251 48.786) (width 0.25) (layer "F.Cu") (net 19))
 (segment (start 32.2982 47.2591) (end 33.8251 48.786) (width 0.25) (layer "F.Cu") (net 19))
 (segment (start 31.116 41.91) (end 32.2982 43.0922) (width 0.25) (layer "F.Cu") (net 19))
 (segment (start 32.2561 57.0259) (end 32.2561 52.9784) (width 0.25) (layer "F.Cu") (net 17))
 (segment (start 31.116 58.166) (end 32.2561 57.0259) (width 0.25) (layer "F.Cu") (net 17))
 (segment (start 33.4485 51.786) (end 34.772 51.786) (width 0.25) (layer "F.Cu") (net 17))
 (segment (start 32.2561 52.9784) (end 33.4485 51.786) (width 0.25) (layer "F.Cu") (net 17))
 (segment (start 30.8604 66.04) (end 30.7716 65.9512) (width 0.25) (layer "F.Cu") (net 24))
 (segment (start 36.068 58.928) (end 36.068 60.452) (width 0.25) (layer "F.Cu") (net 24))
 (segment (start 32.362 66.04) (end 30.8604 66.04) (width 0.25) (layer "F.Cu") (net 24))
 (via (at 30.7716 65.9512) (size 0.8) (drill 0.4) (layers "F.Cu" "B.Cu") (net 24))
 (via (at 36.068 60.452) (size 0.8) (drill 0.4) (layers "F.Cu" "B.Cu") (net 24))
 (segment (start 34.1043 62.6185) (end 30.7716 65.9512) (width 0.25) (layer "B.Cu") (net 24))
 (segment (start 36.068 60.452) (end 34.1043 62.4157) (width 0.25) (layer "B.Cu") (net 24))
 (segment (start 34.1043 62.4157) (end 34.1043 62.6185) (width 0.25) (layer "B.Cu") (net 24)))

